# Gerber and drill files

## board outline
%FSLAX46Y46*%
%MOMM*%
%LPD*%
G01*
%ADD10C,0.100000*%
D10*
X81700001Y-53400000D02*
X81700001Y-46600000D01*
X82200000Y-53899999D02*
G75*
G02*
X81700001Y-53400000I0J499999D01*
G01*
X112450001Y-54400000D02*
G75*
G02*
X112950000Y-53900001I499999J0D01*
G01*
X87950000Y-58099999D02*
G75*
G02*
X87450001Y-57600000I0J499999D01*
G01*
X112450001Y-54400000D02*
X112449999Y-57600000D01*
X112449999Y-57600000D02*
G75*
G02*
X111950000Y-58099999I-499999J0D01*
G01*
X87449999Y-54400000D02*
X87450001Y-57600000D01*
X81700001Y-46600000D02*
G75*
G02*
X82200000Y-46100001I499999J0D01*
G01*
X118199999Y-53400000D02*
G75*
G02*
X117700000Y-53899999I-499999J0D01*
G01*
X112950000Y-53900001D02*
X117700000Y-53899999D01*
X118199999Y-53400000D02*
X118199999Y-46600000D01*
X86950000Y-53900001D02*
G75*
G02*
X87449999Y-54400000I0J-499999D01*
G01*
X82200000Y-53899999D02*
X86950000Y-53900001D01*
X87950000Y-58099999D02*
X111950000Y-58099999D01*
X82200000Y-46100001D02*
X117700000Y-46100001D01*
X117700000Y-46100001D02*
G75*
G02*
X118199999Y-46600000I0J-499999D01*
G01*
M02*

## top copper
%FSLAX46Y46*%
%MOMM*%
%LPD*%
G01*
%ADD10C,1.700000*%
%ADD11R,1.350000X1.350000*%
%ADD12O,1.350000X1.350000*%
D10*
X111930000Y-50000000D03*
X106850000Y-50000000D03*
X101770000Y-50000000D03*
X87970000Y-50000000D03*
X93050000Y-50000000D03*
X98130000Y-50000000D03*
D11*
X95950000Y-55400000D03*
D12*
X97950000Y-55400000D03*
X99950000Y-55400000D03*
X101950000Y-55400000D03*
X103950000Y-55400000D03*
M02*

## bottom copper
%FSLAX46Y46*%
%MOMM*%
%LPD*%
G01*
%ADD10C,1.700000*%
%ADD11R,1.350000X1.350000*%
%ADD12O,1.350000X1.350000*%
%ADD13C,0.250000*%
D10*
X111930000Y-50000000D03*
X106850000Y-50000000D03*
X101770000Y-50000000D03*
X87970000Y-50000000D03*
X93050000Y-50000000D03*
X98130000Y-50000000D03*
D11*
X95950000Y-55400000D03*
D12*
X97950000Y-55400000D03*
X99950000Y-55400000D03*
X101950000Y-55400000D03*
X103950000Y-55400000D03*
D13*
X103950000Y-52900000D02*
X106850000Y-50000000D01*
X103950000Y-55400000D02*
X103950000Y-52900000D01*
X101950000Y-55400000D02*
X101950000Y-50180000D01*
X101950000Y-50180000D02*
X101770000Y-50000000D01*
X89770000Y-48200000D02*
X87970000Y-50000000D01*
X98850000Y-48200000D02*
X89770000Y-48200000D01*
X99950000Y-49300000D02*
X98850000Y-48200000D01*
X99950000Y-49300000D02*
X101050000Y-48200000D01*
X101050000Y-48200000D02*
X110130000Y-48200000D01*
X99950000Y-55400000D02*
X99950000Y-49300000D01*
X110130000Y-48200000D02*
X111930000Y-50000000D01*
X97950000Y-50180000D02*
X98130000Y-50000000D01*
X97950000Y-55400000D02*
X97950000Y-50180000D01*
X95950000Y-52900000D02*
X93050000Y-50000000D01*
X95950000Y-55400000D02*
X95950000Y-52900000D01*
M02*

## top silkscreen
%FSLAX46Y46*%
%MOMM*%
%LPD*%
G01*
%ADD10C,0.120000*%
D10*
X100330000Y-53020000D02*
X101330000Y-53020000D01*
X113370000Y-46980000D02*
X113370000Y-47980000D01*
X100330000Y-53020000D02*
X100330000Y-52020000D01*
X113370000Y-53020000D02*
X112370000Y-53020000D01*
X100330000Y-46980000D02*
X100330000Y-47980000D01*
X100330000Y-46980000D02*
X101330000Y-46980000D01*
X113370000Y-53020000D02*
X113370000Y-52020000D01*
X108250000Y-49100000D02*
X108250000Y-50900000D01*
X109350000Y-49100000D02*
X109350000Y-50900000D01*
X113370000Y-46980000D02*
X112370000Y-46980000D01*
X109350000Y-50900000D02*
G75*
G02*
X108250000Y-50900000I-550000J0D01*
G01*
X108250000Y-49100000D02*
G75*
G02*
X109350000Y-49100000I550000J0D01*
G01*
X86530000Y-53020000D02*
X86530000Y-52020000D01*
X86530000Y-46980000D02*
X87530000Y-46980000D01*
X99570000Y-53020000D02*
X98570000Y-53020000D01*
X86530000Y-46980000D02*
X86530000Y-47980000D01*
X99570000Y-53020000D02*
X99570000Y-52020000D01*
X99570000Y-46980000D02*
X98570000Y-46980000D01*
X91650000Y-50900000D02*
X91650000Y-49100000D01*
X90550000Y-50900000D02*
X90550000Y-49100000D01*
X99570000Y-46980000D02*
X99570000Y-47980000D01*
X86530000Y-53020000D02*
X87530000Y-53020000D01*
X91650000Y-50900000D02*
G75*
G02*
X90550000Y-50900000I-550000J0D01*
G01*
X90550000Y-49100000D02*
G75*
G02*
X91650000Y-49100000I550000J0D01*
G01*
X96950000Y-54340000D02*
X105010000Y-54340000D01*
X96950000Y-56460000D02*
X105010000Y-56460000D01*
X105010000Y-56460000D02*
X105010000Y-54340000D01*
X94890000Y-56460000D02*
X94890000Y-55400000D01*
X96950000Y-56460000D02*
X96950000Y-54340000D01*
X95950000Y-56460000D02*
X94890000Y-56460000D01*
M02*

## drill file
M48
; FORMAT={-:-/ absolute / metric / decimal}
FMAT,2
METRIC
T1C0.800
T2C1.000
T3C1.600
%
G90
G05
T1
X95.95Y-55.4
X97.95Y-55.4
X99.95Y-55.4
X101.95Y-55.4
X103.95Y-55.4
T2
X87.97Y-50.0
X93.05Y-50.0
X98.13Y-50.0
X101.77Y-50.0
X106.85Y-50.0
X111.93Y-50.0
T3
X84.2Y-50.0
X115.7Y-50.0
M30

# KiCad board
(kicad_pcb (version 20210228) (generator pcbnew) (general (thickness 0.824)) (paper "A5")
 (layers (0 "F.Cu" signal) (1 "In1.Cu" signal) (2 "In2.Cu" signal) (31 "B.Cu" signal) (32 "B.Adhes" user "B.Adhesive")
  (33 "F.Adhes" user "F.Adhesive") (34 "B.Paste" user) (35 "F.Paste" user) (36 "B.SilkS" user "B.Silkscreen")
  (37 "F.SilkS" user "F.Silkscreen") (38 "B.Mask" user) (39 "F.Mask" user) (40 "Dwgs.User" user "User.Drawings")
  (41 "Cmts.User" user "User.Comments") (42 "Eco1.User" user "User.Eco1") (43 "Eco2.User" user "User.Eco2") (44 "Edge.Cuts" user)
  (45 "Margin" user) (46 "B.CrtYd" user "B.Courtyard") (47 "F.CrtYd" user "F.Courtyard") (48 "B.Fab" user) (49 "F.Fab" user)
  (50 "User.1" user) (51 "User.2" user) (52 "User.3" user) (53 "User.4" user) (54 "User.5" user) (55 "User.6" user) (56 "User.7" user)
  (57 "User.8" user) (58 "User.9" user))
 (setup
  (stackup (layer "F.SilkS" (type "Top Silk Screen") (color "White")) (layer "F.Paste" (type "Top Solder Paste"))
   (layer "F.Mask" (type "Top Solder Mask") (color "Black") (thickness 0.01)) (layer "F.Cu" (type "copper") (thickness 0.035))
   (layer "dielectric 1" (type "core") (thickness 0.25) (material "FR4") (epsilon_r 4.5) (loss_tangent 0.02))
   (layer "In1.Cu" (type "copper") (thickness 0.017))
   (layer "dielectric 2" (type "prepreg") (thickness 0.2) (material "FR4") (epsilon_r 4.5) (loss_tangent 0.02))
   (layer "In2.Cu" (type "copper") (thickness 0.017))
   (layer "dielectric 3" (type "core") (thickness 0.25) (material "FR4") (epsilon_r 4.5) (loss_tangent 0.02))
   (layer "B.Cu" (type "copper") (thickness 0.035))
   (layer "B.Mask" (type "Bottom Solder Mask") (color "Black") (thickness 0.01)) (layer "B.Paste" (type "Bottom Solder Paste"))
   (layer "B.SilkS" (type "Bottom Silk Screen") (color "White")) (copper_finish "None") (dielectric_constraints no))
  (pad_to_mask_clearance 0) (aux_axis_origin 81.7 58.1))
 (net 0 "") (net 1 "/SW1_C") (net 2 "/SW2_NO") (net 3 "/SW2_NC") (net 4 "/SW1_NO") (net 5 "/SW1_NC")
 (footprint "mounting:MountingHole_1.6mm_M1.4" (layer "F.Cu") (at 115.7 50)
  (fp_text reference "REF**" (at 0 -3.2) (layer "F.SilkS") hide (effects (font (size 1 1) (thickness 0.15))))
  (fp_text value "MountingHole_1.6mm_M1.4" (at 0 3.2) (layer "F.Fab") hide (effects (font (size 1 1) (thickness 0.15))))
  (pad "" np_thru_hole circle (at 0 0) (locked) (size 1.6 1.6) (drill 1.6) (layers F&B.Cu *.Mask)))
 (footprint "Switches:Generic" (layer "F.Cu") (at 106.85 50 180)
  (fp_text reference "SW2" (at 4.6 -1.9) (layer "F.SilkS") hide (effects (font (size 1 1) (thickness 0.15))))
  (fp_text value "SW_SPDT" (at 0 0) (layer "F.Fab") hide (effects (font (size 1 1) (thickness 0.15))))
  (fp_line (start 6.52 -3.02) (end 5.52 -3.02) (layer "F.SilkS") (width 0.12))
  (fp_line (start -6.52 3.02) (end -6.52 2.02) (layer "F.SilkS") (width 0.12))
  (fp_line (start 6.52 -3.02) (end 6.52 -2.02) (layer "F.SilkS") (width 0.12))
  (fp_line (start -6.52 -3.02) (end -5.52 -3.02) (layer "F.SilkS") (width 0.12))
  (fp_line (start 6.52 3.02) (end 6.52 2.02) (layer "F.SilkS") (width 0.12))
  (fp_line (start 6.52 3.02) (end 5.52 3.02) (layer "F.SilkS") (width 0.12))
  (fp_line (start -6.52 -3.02) (end -6.52 -2.02) (layer "F.SilkS") (width 0.12))
  (fp_line (start -1.4 0.9) (end -1.4 -0.9) (layer "F.SilkS") (width 0.12))
  (fp_line (start -2.5 0.9) (end -2.5 -0.9) (layer "F.SilkS") (width 0.12))
  (fp_line (start -6.52 3.02) (end -5.52 3.02) (layer "F.SilkS") (width 0.12))
  (fp_arc (start -1.95 -0.9) (end -1.4 -0.9) (angle -180) (layer "F.SilkS") (width 0.12))
  (fp_arc (start -1.95 0.9) (end -2.5 0.9) (angle -180) (layer "F.SilkS") (width 0.12))
  (pad "1" thru_hole circle (at -5.08 0 180) (locked) (size 1.7 1.7) (drill 1) (layers *.Cu *.Mask) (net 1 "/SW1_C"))
  (pad "2" thru_hole circle (at 0 0 180) (locked) (size 1.7 1.7) (drill 1) (layers *.Cu *.Mask) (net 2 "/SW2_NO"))
  (pad "3" thru_hole circle (at 5.08 0 180) (locked) (size 1.7 1.7) (drill 1) (layers *.Cu *.Mask) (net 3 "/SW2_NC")))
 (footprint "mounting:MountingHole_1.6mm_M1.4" (layer "F.Cu") (at 84.2 50)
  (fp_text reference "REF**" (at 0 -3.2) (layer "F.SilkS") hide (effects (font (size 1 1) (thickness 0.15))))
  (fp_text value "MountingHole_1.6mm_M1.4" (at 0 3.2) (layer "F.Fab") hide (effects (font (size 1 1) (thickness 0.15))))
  (pad "" np_thru_hole circle (at 0 0) (locked) (size 1.6 1.6) (drill 1.6) (layers F&B.Cu *.Mask)))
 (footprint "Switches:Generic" (layer "F.Cu") (at 93.05 50)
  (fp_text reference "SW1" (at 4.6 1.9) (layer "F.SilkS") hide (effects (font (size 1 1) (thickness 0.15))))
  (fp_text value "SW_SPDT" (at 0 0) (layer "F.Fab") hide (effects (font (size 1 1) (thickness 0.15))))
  (fp_line (start -6.52 3.02) (end -6.52 2.02) (layer "F.SilkS") (width 0.12))
  (fp_line (start -6.52 -3.02) (end -5.52 -3.02) (layer "F.SilkS") (width 0.12))
  (fp_line (start 6.52 3.02) (end 5.52 3.02) (layer "F.SilkS") (width 0.12))
  (fp_line (start -6.52 -3.02) (end -6.52 -2.02) (layer "F.SilkS") (width 0.12))
  (fp_line (start 6.52 3.02) (end 6.52 2.02) (layer "F.SilkS") (width 0.12))
  (fp_line (start 6.52 -3.02) (end 5.52 -3.02) (layer "F.SilkS") (width 0.12))
  (fp_line (start -1.4 0.9) (end -1.4 -0.9) (layer "F.SilkS") (width 0.12))
  (fp_line (start -2.5 0.9) (end -2.5 -0.9) (layer "F.SilkS") (width 0.12))
  (fp_line (start 6.52 -3.02) (end 6.52 -2.02) (layer "F.SilkS") (width 0.12))
  (fp_line (start -6.52 3.02) (end -5.52 3.02) (layer "F.SilkS") (width 0.12))
  (fp_arc (start -1.95 0.9) (end -2.5 0.9) (angle -180) (layer "F.SilkS") (width 0.12))
  (fp_arc (start -1.95 -0.9) (end -1.4 -0.9) (angle -180) (layer "F.SilkS") (width 0.12))
  (pad "1" thru_hole circle (at -5.08 0) (locked) (size 1.7 1.7) (drill 1) (layers *.Cu *.Mask) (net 1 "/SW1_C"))
  (pad "2" thru_hole circle (at 0 0) (locked) (size 1.7 1.7) (drill 1) (layers *.Cu *.Mask) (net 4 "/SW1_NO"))
  (pad "3" thru_hole circle (at 5.08 0) (locked) (size 1.7 1.7) (drill 1) (layers *.Cu *.Mask) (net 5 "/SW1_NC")))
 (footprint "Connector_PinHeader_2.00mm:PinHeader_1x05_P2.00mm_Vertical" (layer "F.Cu") (at 95.95 55.4 90)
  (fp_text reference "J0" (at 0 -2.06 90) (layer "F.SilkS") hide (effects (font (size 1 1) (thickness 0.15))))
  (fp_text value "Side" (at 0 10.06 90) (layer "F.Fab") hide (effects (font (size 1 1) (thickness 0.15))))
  (fp_line (start 1.06 1) (end 1.06 9.06) (layer "F.SilkS") (width 0.12))
  (fp_line (start -1.06 1) (end -1.06 9.06) (layer "F.SilkS") (width 0.12))
  (fp_line (start -1.06 9.06) (end 1.06 9.06) (layer "F.SilkS") (width 0.12))
  (fp_line (start -1.06 -1.06) (end 0 -1.06) (layer "F.SilkS") (width 0.12))
  (fp_line (start -1.06 1) (end 1.06 1) (layer "F.SilkS") (width 0.12))
  (fp_line (start -1.06 0) (end -1.06 -1.06) (layer "F.SilkS") (width 0.12))
  (pad "1" thru_hole rect (at 0 0 90) (locked) (size 1.35 1.35) (drill 0.8) (layers *.Cu *.Mask) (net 4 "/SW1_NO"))
  (pad "2" thru_hole oval (at 0 2 90) (locked) (size 1.35 1.35) (drill 0.8) (layers *.Cu *.Mask) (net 5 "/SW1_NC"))
  (pad "3" thru_hole oval (at 0 4 90) (locked) (size 1.35 1.35) (drill 0.8) (layers *.Cu *.Mask) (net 1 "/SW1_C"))
  (pad "4" thru_hole oval (at 0 6 90) (locked) (size 1.35 1.35) (drill 0.8) (layers *.Cu *.Mask) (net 3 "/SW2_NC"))
  (pad "5" thru_hole oval (at 0 8 90) (locked) (size 1.35 1.35) (drill 0.8) (layers *.Cu *.Mask) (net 2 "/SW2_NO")))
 (gr_line (start 81.700001 53.4) (end 81.700001 46.6) (layer "Edge.Cuts") (width 0.1))
 (gr_arc (start 82.2 53.4) (end 82.2 53.899999) (angle 90) (layer "Edge.Cuts") (width 0.1))
 (gr_arc (start 112.95 54.4) (end 112.450001 54.4) (angle 90) (layer "Edge.Cuts") (width 0.1))
 (gr_arc (start 87.95 57.6) (end 87.95 58.099999) (angle 90) (layer "Edge.Cuts") (width 0.1))
 (gr_line (start 112.450001 54.4) (end 112.449999 57.6) (layer "Edge.Cuts") (width 0.1))
 (gr_arc (start 111.95 57.6) (end 112.449999 57.6) (angle 90) (layer "Edge.Cuts") (width 0.1))
 (gr_line (start 87.449999 54.4) (end 87.450001 57.6) (layer "Edge.Cuts") (width 0.1))
 (gr_arc (start 82.2 46.6) (end 81.700001 46.6) (angle 90) (layer "Edge.Cuts") (width 0.1))
 (gr_arc (start 117.7 53.4) (end 118.199999 53.4) (angle 90) (layer "Edge.Cuts") (width 0.1))
 (gr_line (start 112.95 53.900001) (end 117.7 53.899999) (layer "Edge.Cuts") (width 0.1))
 (gr_line (start 118.199999 53.4) (end 118.199999 46.6) (layer "Edge.Cuts") (width 0.1))
 (gr_arc (start 86.95 54.4) (end 86.95 53.900001) (angle 90) (layer "Edge.Cuts") (width 0.1))
 (gr_line (start 82.2 53.899999) (end 86.95 53.900001) (layer "Edge.Cuts") (width 0.1))
 (gr_line (start 87.95 58.099999) (end 111.95 58.099999) (layer "Edge.Cuts") (width 0.1))
 (gr_line (start 82.2 46.100001) (end 117.7 46.100001) (layer "Edge.Cuts") (width 0.1))
 (gr_arc (start 117.7 46.6) (end 117.7 46.100001) (angle 90) (layer "Edge.Cuts") (width 0.1))
 (segment (start 103.95 52.9) (end 106.85 50) (width 0.25) (layer "B.Cu") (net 2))
 (segment (start 103.95 55.4) (end 103.95 52.9) (width 0.25) (layer "B.Cu") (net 2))
 (segment (start 101.95 55.4) (end 101.95 50.18) (width 0.25) (layer "B.Cu") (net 3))
 (segment (start 101.95 50.18) (end 101.77 50) (width 0.25) (layer "B.Cu") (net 3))
 (segment (start 89.77 48.2) (end 87.97 50) (width 0.25) (layer "B.Cu") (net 1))
 (segment (start 98.85 48.2) (end 89.77 48.2) (width 0.25) (layer "B.Cu") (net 1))
 (segment (start 99.95 49.3) (end 98.85 48.2) (width 0.25) (layer "B.Cu") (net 1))
 (segment (start 99.95 49.3) (end 101.05 48.2) (width 0.25) (layer "B.Cu") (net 1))
 (segment (start 101.05 48.2) (end 110.13 48.2) (width 0.25) (layer "B.Cu") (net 1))
 (segment (start 99.95 55.4) (end 99.95 49.3) (width 0.25) (layer "B.Cu") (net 1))
 (segment (start 110.13 48.2) (end 111.93 50) (width 0.25) (layer "B.Cu") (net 1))
 (segment (start 97.95 50.18) (end 98.13 50) (width 0.25) (layer "B.Cu") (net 5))
 (segment (start 97.95 55.4) (end 97.95 50.18) (width 0.25) (layer "B.Cu") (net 5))
 (segment (start 95.95 52.9) (end 93.05 50) (width 0.25) (layer "B.Cu") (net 4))
 (segment (start 95.95 55.4) (end 95.95 52.9) (width 0.25) (layer "B.Cu") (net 4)))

